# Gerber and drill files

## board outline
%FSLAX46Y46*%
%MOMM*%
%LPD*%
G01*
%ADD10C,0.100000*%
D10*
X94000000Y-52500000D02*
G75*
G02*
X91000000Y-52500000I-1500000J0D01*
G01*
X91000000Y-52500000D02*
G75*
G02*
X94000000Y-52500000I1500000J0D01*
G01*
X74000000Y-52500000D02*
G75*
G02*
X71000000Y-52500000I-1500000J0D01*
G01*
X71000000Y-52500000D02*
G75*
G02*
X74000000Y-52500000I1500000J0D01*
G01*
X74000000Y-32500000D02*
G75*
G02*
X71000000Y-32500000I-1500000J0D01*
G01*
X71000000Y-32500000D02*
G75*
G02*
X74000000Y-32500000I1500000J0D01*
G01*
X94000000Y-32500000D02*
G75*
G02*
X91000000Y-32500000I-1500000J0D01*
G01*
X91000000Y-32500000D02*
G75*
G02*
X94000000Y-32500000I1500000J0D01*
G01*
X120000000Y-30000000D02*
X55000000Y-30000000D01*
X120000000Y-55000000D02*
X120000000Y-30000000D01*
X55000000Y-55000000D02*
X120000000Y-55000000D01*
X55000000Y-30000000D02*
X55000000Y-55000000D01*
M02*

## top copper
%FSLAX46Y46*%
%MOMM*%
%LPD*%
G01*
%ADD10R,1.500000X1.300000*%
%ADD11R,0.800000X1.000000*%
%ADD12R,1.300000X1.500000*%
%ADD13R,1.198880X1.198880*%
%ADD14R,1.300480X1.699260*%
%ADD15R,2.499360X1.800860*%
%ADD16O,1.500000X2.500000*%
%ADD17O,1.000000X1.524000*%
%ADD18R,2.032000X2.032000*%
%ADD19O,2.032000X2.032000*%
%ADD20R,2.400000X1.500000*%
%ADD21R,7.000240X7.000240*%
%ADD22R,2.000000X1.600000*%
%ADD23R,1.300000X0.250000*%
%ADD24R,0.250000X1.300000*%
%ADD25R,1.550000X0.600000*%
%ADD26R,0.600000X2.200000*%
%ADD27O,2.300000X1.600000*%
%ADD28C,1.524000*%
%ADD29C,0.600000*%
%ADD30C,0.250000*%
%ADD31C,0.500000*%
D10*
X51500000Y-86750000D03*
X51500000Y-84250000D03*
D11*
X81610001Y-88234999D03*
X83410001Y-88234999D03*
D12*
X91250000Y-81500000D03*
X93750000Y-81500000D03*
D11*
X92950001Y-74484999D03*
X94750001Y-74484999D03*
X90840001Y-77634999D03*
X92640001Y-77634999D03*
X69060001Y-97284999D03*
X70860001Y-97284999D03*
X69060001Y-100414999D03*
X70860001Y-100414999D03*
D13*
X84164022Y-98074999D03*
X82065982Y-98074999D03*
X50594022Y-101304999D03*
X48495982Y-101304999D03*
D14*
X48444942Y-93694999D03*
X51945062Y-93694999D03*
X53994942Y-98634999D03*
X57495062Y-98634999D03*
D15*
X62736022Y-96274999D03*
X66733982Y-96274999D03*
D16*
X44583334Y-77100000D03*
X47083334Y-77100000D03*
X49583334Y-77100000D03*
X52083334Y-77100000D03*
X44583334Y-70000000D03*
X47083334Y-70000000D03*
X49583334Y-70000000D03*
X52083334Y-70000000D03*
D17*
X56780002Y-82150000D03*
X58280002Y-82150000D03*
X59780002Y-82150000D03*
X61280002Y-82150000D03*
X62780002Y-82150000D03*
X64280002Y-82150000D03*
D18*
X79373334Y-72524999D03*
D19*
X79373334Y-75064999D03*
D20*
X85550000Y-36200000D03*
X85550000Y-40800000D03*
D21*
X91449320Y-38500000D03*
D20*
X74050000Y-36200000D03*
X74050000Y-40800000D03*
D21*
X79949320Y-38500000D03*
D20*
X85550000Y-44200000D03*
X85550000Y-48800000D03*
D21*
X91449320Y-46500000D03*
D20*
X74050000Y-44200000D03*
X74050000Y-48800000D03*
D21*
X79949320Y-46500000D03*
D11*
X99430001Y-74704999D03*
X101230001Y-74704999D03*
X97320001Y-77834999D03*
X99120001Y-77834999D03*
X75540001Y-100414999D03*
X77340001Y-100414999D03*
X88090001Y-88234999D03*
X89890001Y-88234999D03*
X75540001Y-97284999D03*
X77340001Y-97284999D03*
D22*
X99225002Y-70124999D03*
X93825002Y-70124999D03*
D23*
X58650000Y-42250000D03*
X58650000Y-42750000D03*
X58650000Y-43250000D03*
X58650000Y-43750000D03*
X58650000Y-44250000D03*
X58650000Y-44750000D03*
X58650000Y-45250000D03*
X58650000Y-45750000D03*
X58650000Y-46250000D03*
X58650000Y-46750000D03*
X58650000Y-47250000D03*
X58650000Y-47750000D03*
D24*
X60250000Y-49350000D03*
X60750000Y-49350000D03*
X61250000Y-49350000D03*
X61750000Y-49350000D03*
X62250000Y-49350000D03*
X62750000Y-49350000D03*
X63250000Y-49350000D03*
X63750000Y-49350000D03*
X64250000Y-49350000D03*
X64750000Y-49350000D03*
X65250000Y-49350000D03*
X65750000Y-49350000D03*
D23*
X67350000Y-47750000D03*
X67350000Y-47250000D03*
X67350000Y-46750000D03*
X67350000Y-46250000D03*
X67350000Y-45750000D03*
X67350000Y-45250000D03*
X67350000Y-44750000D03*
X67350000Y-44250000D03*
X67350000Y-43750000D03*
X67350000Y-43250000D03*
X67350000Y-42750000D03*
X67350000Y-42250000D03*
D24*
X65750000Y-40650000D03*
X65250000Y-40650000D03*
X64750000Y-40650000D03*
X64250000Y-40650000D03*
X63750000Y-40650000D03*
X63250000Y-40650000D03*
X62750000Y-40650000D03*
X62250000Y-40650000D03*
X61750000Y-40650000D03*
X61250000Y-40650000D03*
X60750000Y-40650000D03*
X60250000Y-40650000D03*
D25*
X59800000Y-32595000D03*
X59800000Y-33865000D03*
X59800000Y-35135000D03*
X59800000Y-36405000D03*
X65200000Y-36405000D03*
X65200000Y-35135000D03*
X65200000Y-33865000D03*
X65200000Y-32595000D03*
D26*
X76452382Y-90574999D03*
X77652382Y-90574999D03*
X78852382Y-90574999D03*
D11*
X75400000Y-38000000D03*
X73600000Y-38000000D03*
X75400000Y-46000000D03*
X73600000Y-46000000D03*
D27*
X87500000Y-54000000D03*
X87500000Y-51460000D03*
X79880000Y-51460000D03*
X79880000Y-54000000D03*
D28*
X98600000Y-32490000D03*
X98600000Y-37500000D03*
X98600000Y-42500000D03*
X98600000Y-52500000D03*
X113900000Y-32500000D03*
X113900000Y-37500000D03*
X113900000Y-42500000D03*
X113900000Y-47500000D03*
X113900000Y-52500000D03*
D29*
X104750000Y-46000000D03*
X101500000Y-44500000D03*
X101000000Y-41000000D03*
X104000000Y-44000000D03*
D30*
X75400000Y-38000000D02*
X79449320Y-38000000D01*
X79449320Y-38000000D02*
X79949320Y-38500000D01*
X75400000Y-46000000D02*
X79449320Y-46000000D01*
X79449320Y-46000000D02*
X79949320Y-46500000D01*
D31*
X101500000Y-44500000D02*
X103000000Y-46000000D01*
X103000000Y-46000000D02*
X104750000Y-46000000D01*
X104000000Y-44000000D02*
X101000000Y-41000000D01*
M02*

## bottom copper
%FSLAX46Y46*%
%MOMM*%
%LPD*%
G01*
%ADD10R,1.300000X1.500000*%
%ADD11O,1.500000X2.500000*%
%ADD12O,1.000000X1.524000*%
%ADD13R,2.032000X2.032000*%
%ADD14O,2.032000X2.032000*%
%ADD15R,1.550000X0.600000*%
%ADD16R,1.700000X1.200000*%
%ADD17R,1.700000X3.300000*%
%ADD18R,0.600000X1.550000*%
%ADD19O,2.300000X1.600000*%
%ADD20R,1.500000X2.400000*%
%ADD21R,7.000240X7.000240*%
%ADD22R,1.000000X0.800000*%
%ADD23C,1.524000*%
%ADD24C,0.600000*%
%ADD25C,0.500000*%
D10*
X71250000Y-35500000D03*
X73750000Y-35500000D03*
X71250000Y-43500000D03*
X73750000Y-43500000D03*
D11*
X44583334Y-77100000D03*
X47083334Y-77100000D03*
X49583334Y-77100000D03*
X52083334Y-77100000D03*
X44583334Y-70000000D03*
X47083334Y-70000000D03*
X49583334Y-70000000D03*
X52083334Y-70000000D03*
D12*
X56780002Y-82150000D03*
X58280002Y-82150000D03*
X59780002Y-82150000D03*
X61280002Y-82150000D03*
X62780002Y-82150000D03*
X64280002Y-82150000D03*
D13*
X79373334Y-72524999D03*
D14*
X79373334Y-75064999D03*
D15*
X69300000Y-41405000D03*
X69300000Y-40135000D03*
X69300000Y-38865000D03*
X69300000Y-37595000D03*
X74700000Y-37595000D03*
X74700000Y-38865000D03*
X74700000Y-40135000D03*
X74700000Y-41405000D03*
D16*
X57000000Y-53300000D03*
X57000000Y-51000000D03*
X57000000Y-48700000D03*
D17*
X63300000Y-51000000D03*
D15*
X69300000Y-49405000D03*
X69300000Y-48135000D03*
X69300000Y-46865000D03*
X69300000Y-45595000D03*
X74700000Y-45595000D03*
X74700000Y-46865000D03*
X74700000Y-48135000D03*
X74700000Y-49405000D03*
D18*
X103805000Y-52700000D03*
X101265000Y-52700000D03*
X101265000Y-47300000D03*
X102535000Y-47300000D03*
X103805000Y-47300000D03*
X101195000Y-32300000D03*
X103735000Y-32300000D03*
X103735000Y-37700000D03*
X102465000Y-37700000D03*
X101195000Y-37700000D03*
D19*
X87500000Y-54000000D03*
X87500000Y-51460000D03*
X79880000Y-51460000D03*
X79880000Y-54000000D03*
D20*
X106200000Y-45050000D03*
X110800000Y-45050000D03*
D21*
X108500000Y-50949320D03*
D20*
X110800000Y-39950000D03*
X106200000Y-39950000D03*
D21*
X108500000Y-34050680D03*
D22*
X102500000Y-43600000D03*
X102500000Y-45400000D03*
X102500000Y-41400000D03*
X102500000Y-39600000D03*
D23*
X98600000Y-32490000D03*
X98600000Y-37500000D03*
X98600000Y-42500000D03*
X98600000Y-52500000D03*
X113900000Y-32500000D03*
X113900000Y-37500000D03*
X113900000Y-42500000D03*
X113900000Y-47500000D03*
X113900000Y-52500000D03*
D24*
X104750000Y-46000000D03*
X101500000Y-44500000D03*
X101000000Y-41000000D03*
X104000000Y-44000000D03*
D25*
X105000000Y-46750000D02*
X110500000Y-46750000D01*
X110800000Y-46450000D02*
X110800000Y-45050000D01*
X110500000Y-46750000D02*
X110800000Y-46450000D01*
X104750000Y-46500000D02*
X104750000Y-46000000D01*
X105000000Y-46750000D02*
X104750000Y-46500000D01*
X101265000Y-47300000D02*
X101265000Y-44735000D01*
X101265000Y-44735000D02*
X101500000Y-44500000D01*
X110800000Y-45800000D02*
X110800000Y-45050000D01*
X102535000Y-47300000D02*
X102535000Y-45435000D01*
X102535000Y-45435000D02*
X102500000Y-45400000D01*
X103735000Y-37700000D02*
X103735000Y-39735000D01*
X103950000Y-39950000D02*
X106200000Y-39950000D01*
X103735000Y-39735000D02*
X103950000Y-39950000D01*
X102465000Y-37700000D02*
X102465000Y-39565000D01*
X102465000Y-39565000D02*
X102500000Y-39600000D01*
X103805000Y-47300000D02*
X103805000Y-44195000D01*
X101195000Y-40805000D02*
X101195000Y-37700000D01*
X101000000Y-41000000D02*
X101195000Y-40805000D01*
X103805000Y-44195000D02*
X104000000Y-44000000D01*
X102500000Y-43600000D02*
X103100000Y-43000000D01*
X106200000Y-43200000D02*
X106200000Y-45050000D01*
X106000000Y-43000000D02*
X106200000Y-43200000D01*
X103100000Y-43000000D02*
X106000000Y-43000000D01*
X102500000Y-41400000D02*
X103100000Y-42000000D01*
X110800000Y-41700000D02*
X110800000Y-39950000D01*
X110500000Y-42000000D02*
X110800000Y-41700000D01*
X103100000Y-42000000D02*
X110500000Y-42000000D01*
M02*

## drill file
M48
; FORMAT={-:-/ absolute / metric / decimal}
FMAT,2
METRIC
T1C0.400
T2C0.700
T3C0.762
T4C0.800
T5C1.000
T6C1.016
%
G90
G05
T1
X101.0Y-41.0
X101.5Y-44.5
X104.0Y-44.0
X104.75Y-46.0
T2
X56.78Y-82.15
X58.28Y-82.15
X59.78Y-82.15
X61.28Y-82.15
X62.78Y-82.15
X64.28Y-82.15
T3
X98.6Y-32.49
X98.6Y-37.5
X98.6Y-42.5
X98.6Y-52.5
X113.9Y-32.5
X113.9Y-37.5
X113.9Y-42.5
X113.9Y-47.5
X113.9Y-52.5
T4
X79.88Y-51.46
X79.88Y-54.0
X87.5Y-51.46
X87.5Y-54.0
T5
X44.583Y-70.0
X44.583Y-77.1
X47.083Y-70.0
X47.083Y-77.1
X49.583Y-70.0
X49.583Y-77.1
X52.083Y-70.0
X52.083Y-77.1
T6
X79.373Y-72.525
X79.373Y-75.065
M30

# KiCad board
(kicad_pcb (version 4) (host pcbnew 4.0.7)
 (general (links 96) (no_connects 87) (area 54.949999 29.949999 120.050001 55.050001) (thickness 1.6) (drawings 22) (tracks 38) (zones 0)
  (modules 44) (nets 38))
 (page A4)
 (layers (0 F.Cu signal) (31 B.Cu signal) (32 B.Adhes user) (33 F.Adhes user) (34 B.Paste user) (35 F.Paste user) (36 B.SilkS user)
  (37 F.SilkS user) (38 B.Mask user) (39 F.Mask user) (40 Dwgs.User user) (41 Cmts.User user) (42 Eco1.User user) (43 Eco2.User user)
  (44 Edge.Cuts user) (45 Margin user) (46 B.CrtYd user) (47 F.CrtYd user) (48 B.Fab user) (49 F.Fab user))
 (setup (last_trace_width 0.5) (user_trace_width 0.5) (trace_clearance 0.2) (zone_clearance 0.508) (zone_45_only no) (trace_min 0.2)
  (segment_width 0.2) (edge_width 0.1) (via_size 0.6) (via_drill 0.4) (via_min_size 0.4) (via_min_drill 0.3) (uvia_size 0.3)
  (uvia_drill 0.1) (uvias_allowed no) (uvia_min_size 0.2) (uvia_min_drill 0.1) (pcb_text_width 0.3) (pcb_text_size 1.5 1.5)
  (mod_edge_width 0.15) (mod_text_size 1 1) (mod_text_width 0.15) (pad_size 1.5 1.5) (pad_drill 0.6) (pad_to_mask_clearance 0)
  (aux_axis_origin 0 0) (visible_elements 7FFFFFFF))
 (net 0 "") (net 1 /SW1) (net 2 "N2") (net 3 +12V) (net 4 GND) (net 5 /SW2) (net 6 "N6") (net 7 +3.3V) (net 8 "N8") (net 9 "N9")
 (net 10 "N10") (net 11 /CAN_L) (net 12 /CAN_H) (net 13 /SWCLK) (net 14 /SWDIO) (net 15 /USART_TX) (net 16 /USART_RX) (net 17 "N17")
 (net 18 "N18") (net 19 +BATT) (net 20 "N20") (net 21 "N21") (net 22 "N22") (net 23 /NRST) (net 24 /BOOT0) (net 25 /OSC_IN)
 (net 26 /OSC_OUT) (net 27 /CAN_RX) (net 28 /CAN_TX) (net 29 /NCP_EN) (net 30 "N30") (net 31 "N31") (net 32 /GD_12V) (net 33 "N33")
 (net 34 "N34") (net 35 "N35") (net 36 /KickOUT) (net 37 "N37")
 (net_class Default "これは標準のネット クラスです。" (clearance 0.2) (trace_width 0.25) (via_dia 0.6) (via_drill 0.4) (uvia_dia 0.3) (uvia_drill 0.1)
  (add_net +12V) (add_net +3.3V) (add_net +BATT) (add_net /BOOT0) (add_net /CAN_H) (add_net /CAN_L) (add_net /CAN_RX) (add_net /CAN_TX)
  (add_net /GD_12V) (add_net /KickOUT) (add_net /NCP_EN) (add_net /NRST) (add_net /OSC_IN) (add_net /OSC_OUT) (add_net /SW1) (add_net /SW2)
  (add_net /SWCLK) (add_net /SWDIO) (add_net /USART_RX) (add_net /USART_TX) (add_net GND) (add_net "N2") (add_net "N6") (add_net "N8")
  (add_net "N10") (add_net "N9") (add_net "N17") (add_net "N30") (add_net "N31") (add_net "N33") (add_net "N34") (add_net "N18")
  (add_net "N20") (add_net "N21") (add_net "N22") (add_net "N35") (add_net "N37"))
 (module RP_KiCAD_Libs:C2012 (layer B.Cu) (at 72.5 35.5)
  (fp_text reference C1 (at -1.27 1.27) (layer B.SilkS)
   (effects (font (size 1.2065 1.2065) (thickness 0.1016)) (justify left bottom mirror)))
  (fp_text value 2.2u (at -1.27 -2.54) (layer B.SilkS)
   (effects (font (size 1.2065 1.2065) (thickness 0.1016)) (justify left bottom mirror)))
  (pad 1 smd rect (at -1.25 0) (size 1.3 1.5) (layers B.Cu B.Paste B.Mask) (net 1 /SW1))
  (pad 2 smd rect (at 1.25 0) (size 1.3 1.5) (layers B.Cu B.Paste B.Mask) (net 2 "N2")))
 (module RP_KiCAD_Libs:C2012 (layer F.Cu) (at 51.5 85.5 90)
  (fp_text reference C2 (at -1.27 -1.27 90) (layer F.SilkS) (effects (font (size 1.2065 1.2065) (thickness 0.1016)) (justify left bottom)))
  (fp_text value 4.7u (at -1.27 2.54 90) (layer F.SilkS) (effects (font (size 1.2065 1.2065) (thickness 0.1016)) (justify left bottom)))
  (pad 1 smd rect (at -1.25 0 90) (size 1.3 1.5) (layers F.Cu F.Paste F.Mask) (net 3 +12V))
  (pad 2 smd rect (at 1.25 0 90) (size 1.3 1.5) (layers F.Cu F.Paste F.Mask) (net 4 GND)))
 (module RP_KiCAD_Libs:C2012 (layer B.Cu) (at 72.5 43.5)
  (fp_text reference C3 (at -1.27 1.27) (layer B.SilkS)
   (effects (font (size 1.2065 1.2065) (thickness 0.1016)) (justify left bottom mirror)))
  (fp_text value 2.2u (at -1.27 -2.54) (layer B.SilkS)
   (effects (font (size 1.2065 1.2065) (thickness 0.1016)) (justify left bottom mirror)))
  (pad 1 smd rect (at -1.25 0) (size 1.3 1.5) (layers B.Cu B.Paste B.Mask) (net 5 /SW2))
  (pad 2 smd rect (at 1.25 0) (size 1.3 1.5) (layers B.Cu B.Paste B.Mask) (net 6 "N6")))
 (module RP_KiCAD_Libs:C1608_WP (layer F.Cu) (at 82.510001 88.234999)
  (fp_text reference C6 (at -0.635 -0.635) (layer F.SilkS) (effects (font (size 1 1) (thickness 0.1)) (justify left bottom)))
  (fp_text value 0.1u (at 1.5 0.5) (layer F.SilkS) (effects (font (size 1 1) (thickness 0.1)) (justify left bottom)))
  (pad 1 smd rect (at -0.9 0) (size 0.8 1) (layers F.Cu F.Paste F.Mask) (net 4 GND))
  (pad 2 smd rect (at 0.9 0) (size 0.8 1) (layers F.Cu F.Paste F.Mask) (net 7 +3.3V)))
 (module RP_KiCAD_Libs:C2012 (layer F.Cu) (at 92.5 81.5)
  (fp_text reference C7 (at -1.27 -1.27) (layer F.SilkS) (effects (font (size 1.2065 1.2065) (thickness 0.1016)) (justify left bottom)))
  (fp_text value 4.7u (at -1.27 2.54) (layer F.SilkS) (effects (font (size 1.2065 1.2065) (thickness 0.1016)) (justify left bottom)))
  (pad 1 smd rect (at -1.25 0) (size 1.3 1.5) (layers F.Cu F.Paste F.Mask) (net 7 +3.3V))
  (pad 2 smd rect (at 1.25 0) (size 1.3 1.5) (layers F.Cu F.Paste F.Mask) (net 4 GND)))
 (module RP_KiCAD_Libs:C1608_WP (layer F.Cu) (at 93.850001 74.484999)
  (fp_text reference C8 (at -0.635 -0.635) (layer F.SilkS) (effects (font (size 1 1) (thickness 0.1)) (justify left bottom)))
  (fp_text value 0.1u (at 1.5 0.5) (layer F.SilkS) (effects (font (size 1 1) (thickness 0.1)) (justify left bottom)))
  (pad 1 smd rect (at -0.9 0) (size 0.8 1) (layers F.Cu F.Paste F.Mask) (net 4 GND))
  (pad 2 smd rect (at 0.9 0) (size 0.8 1) (layers F.Cu F.Paste F.Mask) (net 7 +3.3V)))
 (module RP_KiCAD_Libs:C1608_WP (layer F.Cu) (at 91.740001 77.634999)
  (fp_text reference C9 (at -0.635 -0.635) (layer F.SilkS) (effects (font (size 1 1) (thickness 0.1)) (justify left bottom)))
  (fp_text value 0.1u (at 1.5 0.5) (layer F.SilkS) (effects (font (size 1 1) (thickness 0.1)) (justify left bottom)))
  (pad 1 smd rect (at -0.9 0) (size 0.8 1) (layers F.Cu F.Paste F.Mask) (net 4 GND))
  (pad 2 smd rect (at 0.9 0) (size 0.8 1) (layers F.Cu F.Paste F.Mask) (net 7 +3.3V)))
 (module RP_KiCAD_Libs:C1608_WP (layer F.Cu) (at 69.960001 97.284999)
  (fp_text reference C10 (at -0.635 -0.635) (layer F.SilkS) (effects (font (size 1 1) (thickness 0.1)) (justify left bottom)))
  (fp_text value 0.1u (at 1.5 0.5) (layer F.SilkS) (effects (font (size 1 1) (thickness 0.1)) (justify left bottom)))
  (pad 1 smd rect (at -0.9 0) (size 0.8 1) (layers F.Cu F.Paste F.Mask) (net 4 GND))
  (pad 2 smd rect (at 0.9 0) (size 0.8 1) (layers F.Cu F.Paste F.Mask) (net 7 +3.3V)))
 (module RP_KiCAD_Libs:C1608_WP (layer F.Cu) (at 69.960001 100.414999)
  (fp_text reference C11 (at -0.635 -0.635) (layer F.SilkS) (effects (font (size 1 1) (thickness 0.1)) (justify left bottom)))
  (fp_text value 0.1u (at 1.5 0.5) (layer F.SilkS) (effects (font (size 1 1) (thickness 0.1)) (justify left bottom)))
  (pad 1 smd rect (at -0.9 0) (size 0.8 1) (layers F.Cu F.Paste F.Mask) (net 4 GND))
  (pad 2 smd rect (at 0.9 0) (size 0.8 1) (layers F.Cu F.Paste F.Mask) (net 7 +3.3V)))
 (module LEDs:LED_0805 (layer F.Cu) (at 83.115002 98.074999)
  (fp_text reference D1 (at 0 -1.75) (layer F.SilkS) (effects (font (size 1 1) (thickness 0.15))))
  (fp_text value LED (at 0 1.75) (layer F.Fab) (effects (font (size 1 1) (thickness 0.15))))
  (pad 1 smd rect (at 1.04902 0 180) (size 1.19888 1.19888) (layers F.Cu F.Paste F.Mask) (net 7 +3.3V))
  (pad 2 smd rect (at -1.04902 0 180) (size 1.19888 1.19888) (layers F.Cu F.Paste F.Mask) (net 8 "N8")))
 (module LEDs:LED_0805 (layer F.Cu) (at 49.545002 101.304999)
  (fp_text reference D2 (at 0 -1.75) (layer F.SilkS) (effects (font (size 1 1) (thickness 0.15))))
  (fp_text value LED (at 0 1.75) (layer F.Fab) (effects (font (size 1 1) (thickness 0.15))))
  (pad 1 smd rect (at 1.04902 0 180) (size 1.19888 1.19888) (layers F.Cu F.Paste F.Mask))
  (pad 2 smd rect (at -1.04902 0 180) (size 1.19888 1.19888) (layers F.Cu F.Paste F.Mask) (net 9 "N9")))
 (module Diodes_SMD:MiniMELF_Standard (layer F.Cu) (at 50.195002 93.694999)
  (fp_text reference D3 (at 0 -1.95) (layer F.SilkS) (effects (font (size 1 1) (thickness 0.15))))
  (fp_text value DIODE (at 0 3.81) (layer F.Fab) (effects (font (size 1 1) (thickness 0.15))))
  (pad 1 smd rect (at -1.75006 0) (size 1.30048 1.69926) (layers F.Cu F.Paste F.Mask) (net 2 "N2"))
  (pad 2 smd rect (at 1.75006 0) (size 1.30048 1.69926) (layers F.Cu F.Paste F.Mask) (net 3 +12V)))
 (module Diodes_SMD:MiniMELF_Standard (layer F.Cu) (at 55.745002 98.634999)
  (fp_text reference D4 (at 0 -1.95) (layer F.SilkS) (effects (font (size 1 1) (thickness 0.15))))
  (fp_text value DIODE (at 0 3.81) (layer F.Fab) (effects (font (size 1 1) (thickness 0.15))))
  (pad 1 smd rect (at -1.75006 0) (size 1.30048 1.69926) (layers F.Cu F.Paste F.Mask) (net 6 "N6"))
  (pad 2 smd rect (at 1.75006 0) (size 1.30048 1.69926) (layers F.Cu F.Paste F.Mask) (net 3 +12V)))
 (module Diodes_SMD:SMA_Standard (layer F.Cu) (at 64.735002 96.274999)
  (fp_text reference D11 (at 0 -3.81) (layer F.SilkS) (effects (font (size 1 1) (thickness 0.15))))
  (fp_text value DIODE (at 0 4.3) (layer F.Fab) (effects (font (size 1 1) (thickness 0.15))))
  (pad 1 smd rect (at -1.99898 0) (size 2.49936 1.80086) (layers F.Cu F.Paste F.Mask) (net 3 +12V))
  (pad 2 smd rect (at 1.99898 0) (size 2.49936 1.80086) (layers F.Cu F.Paste F.Mask) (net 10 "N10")))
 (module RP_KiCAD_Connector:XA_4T (layer F.Cu) (at 44.583334 77.1)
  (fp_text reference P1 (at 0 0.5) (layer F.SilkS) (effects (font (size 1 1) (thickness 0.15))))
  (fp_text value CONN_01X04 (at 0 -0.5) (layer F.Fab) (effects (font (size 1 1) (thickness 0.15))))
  (pad 4 thru_hole oval (at 0 0) (size 1.5 2.5) (drill 1) (layers *.Cu *.Mask F.SilkS) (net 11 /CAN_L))
  (pad 3 thru_hole oval (at 2.5 0) (size 1.5 2.5) (drill 1) (layers *.Cu *.Mask F.SilkS) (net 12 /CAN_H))
  (pad 2 thru_hole oval (at 5 0) (size 1.5 2.5) (drill 1) (layers *.Cu *.Mask F.SilkS) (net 10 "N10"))
  (pad 1 thru_hole oval (at 7.5 0) (size 1.5 2.5) (drill 1) (layers *.Cu *.Mask F.SilkS) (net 4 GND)))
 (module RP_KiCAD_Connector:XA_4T (layer F.Cu) (at 44.583334 70)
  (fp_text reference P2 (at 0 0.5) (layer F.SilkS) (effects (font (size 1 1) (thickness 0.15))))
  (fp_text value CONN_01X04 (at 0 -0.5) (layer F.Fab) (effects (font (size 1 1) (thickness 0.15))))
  (pad 4 thru_hole oval (at 0 0) (size 1.5 2.5) (drill 1) (layers *.Cu *.Mask F.SilkS) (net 11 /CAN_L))
  (pad 3 thru_hole oval (at 2.5 0) (size 1.5 2.5) (drill 1) (layers *.Cu *.Mask F.SilkS) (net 12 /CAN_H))
  (pad 2 thru_hole oval (at 5 0) (size 1.5 2.5) (drill 1) (layers *.Cu *.Mask F.SilkS) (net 10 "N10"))
  (pad 1 thru_hole oval (at 7.5 0) (size 1.5 2.5) (drill 1) (layers *.Cu *.Mask F.SilkS) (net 4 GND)))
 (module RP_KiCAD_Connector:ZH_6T (layer F.Cu) (at 56.780002 82.15)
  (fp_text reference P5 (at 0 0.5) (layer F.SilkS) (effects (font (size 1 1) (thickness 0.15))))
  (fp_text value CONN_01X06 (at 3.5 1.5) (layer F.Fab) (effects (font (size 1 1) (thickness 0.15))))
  (pad 1 thru_hole oval (at 0 0) (size 1 1.524) (drill 0.7) (layers *.Cu *.Mask) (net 4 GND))
  (pad 2 thru_hole oval (at 1.5 0) (size 1 1.524) (drill 0.7) (layers *.Cu *.Mask))
  (pad 3 thru_hole oval (at 3 0) (size 1 1.524) (drill 0.7) (layers *.Cu *.Mask) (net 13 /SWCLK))
  (pad 4 thru_hole oval (at 4.5 0) (size 1 1.524) (drill 0.7) (layers *.Cu *.Mask) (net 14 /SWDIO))
  (pad 5 thru_hole oval (at 6 0) (size 1 1.524) (drill 0.7) (layers *.Cu *.Mask) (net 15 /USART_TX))
  (pad 6 thru_hole oval (at 7.5 0) (size 1 1.524) (drill 0.7) (layers *.Cu *.Mask) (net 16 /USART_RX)))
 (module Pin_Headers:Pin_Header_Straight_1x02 (layer F.Cu) (at 79.373334 72.524999)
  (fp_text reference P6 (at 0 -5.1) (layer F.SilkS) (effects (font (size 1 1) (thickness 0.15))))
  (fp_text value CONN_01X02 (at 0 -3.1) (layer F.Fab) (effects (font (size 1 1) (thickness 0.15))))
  (pad 1 thru_hole rect (at 0 0) (size 2.032 2.032) (drill 1.016) (layers *.Cu *.Mask F.SilkS) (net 12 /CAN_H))
  (pad 2 thru_hole oval (at 0 2.54) (size 2.032 2.032) (drill 1.016) (layers *.Cu *.Mask F.SilkS) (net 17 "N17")))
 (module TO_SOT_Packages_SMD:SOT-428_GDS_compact (layer F.Cu) (at 89 38.5 270)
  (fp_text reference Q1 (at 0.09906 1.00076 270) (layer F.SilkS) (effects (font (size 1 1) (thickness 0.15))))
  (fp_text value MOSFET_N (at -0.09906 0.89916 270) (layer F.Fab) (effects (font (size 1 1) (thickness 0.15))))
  (pad G smd rect (at -2.3 3.45 270) (size 1.5 2.4) (layers F.Cu F.Paste F.Mask) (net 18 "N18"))
  (pad S smd rect (at 2.3 3.45 270) (size 1.5 2.4) (layers F.Cu F.Paste F.Mask) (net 1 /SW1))
  (pad D smd rect (at 0 -2.44932 270) (size 7.00024 7.00024) (layers F.Cu F.Paste F.Mask) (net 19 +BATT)))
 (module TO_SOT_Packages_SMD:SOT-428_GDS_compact (layer F.Cu) (at 77.5 38.5 270)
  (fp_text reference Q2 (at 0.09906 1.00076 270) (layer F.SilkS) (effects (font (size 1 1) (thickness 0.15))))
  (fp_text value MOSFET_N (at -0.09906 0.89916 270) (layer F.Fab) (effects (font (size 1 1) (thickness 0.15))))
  (pad G smd rect (at -2.3 3.45 270) (size 1.5 2.4) (layers F.Cu F.Paste F.Mask) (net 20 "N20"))
  (pad S smd rect (at 2.3 3.45 270) (size 1.5 2.4) (layers F.Cu F.Paste F.Mask) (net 4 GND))
  (pad D smd rect (at 0 -2.44932 270) (size 7.00024 7.00024) (layers F.Cu F.Paste F.Mask) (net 1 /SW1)))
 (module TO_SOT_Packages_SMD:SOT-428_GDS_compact (layer F.Cu) (at 89 46.5 270)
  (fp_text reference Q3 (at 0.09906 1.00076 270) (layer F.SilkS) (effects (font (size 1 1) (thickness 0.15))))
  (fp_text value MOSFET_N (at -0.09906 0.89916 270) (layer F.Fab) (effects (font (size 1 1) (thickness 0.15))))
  (pad G smd rect (at -2.3 3.45 270) (size 1.5 2.4) (layers F.Cu F.Paste F.Mask) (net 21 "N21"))
  (pad S smd rect (at 2.3 3.45 270) (size 1.5 2.4) (layers F.Cu F.Paste F.Mask) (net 5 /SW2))
  (pad D smd rect (at 0 -2.44932 270) (size 7.00024 7.00024) (layers F.Cu F.Paste F.Mask) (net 19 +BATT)))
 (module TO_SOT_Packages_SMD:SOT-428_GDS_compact (layer F.Cu) (at 77.5 46.5 270)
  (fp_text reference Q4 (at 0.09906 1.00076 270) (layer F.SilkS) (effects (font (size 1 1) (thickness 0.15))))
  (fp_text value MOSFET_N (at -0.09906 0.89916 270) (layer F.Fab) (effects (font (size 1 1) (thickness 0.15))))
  (pad G smd rect (at -2.3 3.45 270) (size 1.5 2.4) (layers F.Cu F.Paste F.Mask) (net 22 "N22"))
  (pad S smd rect (at 2.3 3.45 270) (size 1.5 2.4) (layers F.Cu F.Paste F.Mask) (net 4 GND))
  (pad D smd rect (at 0 -2.44932 270) (size 7.00024 7.00024) (layers F.Cu F.Paste F.Mask) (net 5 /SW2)))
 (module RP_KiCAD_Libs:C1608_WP (layer F.Cu) (at 100.330001 74.704999)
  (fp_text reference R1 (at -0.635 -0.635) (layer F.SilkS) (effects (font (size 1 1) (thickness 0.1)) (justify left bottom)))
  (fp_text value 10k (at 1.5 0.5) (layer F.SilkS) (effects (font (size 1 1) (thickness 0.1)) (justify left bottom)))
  (pad 1 smd rect (at -0.9 0) (size 0.8 1) (layers F.Cu F.Paste F.Mask) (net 7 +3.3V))
  (pad 2 smd rect (at 0.9 0) (size 0.8 1) (layers F.Cu F.Paste F.Mask) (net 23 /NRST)))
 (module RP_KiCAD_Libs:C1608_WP (layer F.Cu) (at 98.220001 77.834999)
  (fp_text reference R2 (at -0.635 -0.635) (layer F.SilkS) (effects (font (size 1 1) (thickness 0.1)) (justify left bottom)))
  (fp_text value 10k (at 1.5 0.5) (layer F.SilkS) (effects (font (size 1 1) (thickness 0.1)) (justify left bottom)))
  (pad 1 smd rect (at -0.9 0) (size 0.8 1) (layers F.Cu F.Paste F.Mask) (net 4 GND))
  (pad 2 smd rect (at 0.9 0) (size 0.8 1) (layers F.Cu F.Paste F.Mask) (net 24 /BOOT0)))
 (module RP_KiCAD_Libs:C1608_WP (layer F.Cu) (at 76.440001 100.414999)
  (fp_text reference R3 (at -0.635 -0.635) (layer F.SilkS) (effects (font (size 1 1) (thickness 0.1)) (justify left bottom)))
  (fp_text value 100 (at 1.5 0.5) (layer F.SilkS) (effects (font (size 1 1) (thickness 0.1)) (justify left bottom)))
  (pad 1 smd rect (at -0.9 0) (size 0.8 1) (layers F.Cu F.Paste F.Mask) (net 8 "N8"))
  (pad 2 smd rect (at 0.9 0) (size 0.8 1) (layers F.Cu F.Paste F.Mask) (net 4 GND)))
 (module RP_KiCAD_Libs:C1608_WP (layer F.Cu) (at 88.990001 88.234999)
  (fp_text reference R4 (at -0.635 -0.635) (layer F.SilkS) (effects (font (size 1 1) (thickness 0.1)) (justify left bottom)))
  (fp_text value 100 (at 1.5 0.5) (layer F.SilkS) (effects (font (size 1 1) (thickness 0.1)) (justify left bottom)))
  (pad 1 smd rect (at -0.9 0) (size 0.8 1) (layers F.Cu F.Paste F.Mask) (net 9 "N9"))
  (pad 2 smd rect (at 0.9 0) (size 0.8 1) (layers F.Cu F.Paste F.Mask) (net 4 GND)))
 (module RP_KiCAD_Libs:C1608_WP (layer F.Cu) (at 76.440001 97.284999)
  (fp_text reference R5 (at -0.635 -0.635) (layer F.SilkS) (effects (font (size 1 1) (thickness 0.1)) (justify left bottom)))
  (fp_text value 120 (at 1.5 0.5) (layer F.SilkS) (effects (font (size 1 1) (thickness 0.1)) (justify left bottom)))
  (pad 1 smd rect (at -0.9 0) (size 0.8 1) (layers F.Cu F.Paste F.Mask) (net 11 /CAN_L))
  (pad 2 smd rect (at 0.9 0) (size 0.8 1) (layers F.Cu F.Paste F.Mask) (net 17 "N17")))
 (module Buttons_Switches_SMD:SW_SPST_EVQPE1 (layer F.Cu) (at 96.525002 70.124999)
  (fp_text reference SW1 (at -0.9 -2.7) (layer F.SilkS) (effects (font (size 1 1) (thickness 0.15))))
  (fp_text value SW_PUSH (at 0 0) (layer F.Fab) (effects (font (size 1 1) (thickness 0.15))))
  (pad 2 smd rect (at 2.7 0) (size 2 1.6) (layers F.Cu F.Paste F.Mask) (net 23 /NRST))
  (pad 1 smd rect (at -2.7 0) (size 2 1.6) (layers F.Cu F.Paste F.Mask) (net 4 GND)))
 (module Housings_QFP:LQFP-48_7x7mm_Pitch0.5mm (layer F.Cu) (at 63 45)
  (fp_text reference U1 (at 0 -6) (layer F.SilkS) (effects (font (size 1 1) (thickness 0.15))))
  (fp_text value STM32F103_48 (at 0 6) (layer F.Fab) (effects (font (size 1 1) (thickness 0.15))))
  (pad 1 smd rect (at -4.35 -2.75) (size 1.3 0.25) (layers F.Cu F.Paste F.Mask))
  (pad 2 smd rect (at -4.35 -2.25) (size 1.3 0.25) (layers F.Cu F.Paste F.Mask))
  (pad 3 smd rect (at -4.35 -1.75) (size 1.3 0.25) (layers F.Cu F.Paste F.Mask))
  (pad 4 smd rect (at -4.35 -1.25) (size 1.3 0.25) (layers F.Cu F.Paste F.Mask))
  (pad 5 smd rect (at -4.35 -0.75) (size 1.3 0.25) (layers F.Cu F.Paste F.Mask) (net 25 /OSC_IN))
  (pad 6 smd rect (at -4.35 -0.25) (size 1.3 0.25) (layers F.Cu F.Paste F.Mask) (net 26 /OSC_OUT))
  (pad 7 smd rect (at -4.35 0.25) (size 1.3 0.25) (layers F.Cu F.Paste F.Mask) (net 23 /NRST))
  (pad 8 smd rect (at -4.35 0.75) (size 1.3 0.25) (layers F.Cu F.Paste F.Mask) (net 4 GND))
  (pad 9 smd rect (at -4.35 1.25) (size 1.3 0.25) (layers F.Cu F.Paste F.Mask) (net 7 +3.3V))
  (pad 10 smd rect (at -4.35 1.75) (size 1.3 0.25) (layers F.Cu F.Paste F.Mask))
  (pad 11 smd rect (at -4.35 2.25) (size 1.3 0.25) (layers F.Cu F.Paste F.Mask))
  (pad 12 smd rect (at -4.35 2.75) (size 1.3 0.25) (layers F.Cu F.Paste F.Mask))
  (pad 13 smd rect (at -2.75 4.35 90) (size 1.3 0.25) (layers F.Cu F.Paste F.Mask))
  (pad 14 smd rect (at -2.25 4.35 90) (size 1.3 0.25) (layers F.Cu F.Paste F.Mask))
  (pad 15 smd rect (at -1.75 4.35 90) (size 1.3 0.25) (layers F.Cu F.Paste F.Mask))
  (pad 16 smd rect (at -1.25 4.35 90) (size 1.3 0.25) (layers F.Cu F.Paste F.Mask))
  (pad 17 smd rect (at -0.75 4.35 90) (size 1.3 0.25) (layers F.Cu F.Paste F.Mask))
  (pad 18 smd rect (at -0.25 4.35 90) (size 1.3 0.25) (layers F.Cu F.Paste F.Mask))
  (pad 19 smd rect (at 0.25 4.35 90) (size 1.3 0.25) (layers F.Cu F.Paste F.Mask))
  (pad 20 smd rect (at 0.75 4.35 90) (size 1.3 0.25) (layers F.Cu F.Paste F.Mask))
  (pad 21 smd rect (at 1.25 4.35 90) (size 1.3 0.25) (layers F.Cu F.Paste F.Mask))
  (pad 22 smd rect (at 1.75 4.35 90) (size 1.3 0.25) (layers F.Cu F.Paste F.Mask))
  (pad 23 smd rect (at 2.25 4.35 90) (size 1.3 0.25) (layers F.Cu F.Paste F.Mask) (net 4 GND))
  (pad 24 smd rect (at 2.75 4.35 90) (size 1.3 0.25) (layers F.Cu F.Paste F.Mask) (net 7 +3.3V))
  (pad 25 smd rect (at 4.35 2.75) (size 1.3 0.25) (layers F.Cu F.Paste F.Mask))
  (pad 26 smd rect (at 4.35 2.25) (size 1.3 0.25) (layers F.Cu F.Paste F.Mask))
  (pad 27 smd rect (at 4.35 1.75) (size 1.3 0.25) (layers F.Cu F.Paste F.Mask))
  (pad 28 smd rect (at 4.35 1.25) (size 1.3 0.25) (layers F.Cu F.Paste F.Mask))
  (pad 29 smd rect (at 4.35 0.75) (size 1.3 0.25) (layers F.Cu F.Paste F.Mask))
  (pad 30 smd rect (at 4.35 0.25) (size 1.3 0.25) (layers F.Cu F.Paste F.Mask) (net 15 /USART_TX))
  (pad 31 smd rect (at 4.35 -0.25) (size 1.3 0.25) (layers F.Cu F.Paste F.Mask) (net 16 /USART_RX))
  (pad 32 smd rect (at 4.35 -0.75) (size 1.3 0.25) (layers F.Cu F.Paste F.Mask) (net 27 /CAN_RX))
  (pad 33 smd rect (at 4.35 -1.25) (size 1.3 0.25) (layers F.Cu F.Paste F.Mask) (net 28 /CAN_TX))
  (pad 34 smd rect (at 4.35 -1.75) (size 1.3 0.25) (layers F.Cu F.Paste F.Mask) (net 14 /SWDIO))
  (pad 35 smd rect (at 4.35 -2.25) (size 1.3 0.25) (layers F.Cu F.Paste F.Mask) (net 4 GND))
  (pad 36 smd rect (at 4.35 -2.75) (size 1.3 0.25) (layers F.Cu F.Paste F.Mask) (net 7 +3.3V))
  (pad 37 smd rect (at 2.75 -4.35 90) (size 1.3 0.25) (layers F.Cu F.Paste F.Mask) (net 13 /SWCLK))
  (pad 38 smd rect (at 2.25 -4.35 90) (size 1.3 0.25) (layers F.Cu F.Paste F.Mask))
  (pad 39 smd rect (at 1.75 -4.35 90) (size 1.3 0.25) (layers F.Cu F.Paste F.Mask))
  (pad 40 smd rect (at 1.25 -4.35 90) (size 1.3 0.25) (layers F.Cu F.Paste F.Mask))
  (pad 41 smd rect (at 0.75 -4.35 90) (size 1.3 0.25) (layers F.Cu F.Paste F.Mask))
  (pad 42 smd rect (at 0.25 -4.35 90) (size 1.3 0.25) (layers F.Cu F.Paste F.Mask))
  (pad 43 smd rect (at -0.25 -4.35 90) (size 1.3 0.25) (layers F.Cu F.Paste F.Mask))
  (pad 44 smd rect (at -0.75 -4.35 90) (size 1.3 0.25) (layers F.Cu F.Paste F.Mask) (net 24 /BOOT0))
  (pad 45 smd rect (at -1.25 -4.35 90) (size 1.3 0.25) (layers F.Cu F.Paste F.Mask))
  (pad 46 smd rect (at -1.75 -4.35 90) (size 1.3 0.25) (layers F.Cu F.Paste F.Mask))
  (pad 47 smd rect (at -2.25 -4.35 90) (size 1.3 0.25) (layers F.Cu F.Paste F.Mask) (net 4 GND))
  (pad 48 smd rect (at -2.75 -4.35 90) (size 1.3 0.25) (layers F.Cu F.Paste F.Mask) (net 7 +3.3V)))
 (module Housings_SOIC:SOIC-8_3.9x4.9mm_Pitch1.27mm (layer B.Cu) (at 72 39.5)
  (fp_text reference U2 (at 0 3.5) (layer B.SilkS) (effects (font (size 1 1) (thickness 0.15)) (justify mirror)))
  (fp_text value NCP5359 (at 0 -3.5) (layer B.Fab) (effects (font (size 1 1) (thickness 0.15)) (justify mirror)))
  (pad 1 smd rect (at -2.7 1.905) (size 1.55 0.6) (layers B.Cu B.Paste B.Mask) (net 3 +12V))
  (pad 2 smd rect (at -2.7 0.635) (size 1.55 0.6) (layers B.Cu B.Paste B.Mask))
  (pad 3 smd rect (at -2.7 -0.635) (size 1.55 0.6) (layers B.Cu B.Paste B.Mask) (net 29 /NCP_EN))
  (pad 4 smd rect (at -2.7 -1.905) (size 1.55 0.6) (layers B.Cu B.Paste B.Mask) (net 3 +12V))
  (pad 5 smd rect (at 2.7 -1.905) (size 1.55 0.6) (layers B.Cu B.Paste B.Mask) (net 20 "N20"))
  (pad 6 smd rect (at 2.7 -0.635) (size 1.55 0.6) (layers B.Cu B.Paste B.Mask) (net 4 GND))
  (pad 7 smd rect (at 2.7 0.635) (size 1.55 0.6) (layers B.Cu B.Paste B.Mask) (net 1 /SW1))
  (pad 8 smd rect (at 2.7 1.905) (size 1.55 0.6) (layers B.Cu B.Paste B.Mask) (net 18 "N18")))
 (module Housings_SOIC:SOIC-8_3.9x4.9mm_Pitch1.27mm (layer F.Cu) (at 62.5 34.5)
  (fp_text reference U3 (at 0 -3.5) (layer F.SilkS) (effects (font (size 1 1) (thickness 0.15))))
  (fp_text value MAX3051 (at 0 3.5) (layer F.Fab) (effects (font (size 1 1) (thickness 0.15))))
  (pad 1 smd rect (at -2.7 -1.905) (size 1.55 0.6) (layers F.Cu F.Paste F.Mask) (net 28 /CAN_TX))
  (pad 2 smd rect (at -2.7 -0.635) (size 1.55 0.6) (layers F.Cu F.Paste F.Mask) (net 4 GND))
  (pad 3 smd rect (at -2.7 0.635) (size 1.55 0.6) (layers F.Cu F.Paste F.Mask) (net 7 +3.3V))
  (pad 4 smd rect (at -2.7 1.905) (size 1.55 0.6) (layers F.Cu F.Paste F.Mask) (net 27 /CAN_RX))
  (pad 5 smd rect (at 2.7 1.905) (size 1.55 0.6) (layers F.Cu F.Paste F.Mask) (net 4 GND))
  (pad 6 smd rect (at 2.7 0.635) (size 1.55 0.6) (layers F.Cu F.Paste F.Mask) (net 11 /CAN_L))
  (pad 7 smd rect (at 2.7 -0.635) (size 1.55 0.6) (layers F.Cu F.Paste F.Mask) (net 12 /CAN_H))
  (pad 8 smd rect (at 2.7 -1.905) (size 1.55 0.6) (layers F.Cu F.Paste F.Mask) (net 4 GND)))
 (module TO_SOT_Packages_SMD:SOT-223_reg (layer B.Cu) (at 57 51 90)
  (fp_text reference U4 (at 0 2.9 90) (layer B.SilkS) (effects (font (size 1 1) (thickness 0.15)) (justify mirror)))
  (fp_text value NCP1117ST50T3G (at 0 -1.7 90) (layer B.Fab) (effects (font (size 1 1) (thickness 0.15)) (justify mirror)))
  (pad 1 smd rect (at -2.3 0 90) (size 1.2 1.7) (layers B.Cu B.Paste B.Mask) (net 4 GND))
  (pad 2 smd rect (at 0 0 90) (size 1.2 1.7) (layers B.Cu B.Paste B.Mask) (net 7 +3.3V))
  (pad 3 smd rect (at 2.3 0 90) (size 1.2 1.7) (layers B.Cu B.Paste B.Mask) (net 3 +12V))
  (pad 2 smd rect (at 0 6.3 90) (size 3.3 1.7) (layers B.Cu B.Paste B.Mask) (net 7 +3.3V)))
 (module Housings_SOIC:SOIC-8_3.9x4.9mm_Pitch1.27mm (layer B.Cu) (at 72 47.5)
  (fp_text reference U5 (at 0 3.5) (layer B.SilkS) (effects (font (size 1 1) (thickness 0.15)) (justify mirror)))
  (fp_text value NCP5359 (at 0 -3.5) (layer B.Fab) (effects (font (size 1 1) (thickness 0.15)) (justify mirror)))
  (pad 1 smd rect (at -2.7 1.905) (size 1.55 0.6) (layers B.Cu B.Paste B.Mask) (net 3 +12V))
  (pad 2 smd rect (at -2.7 0.635) (size 1.55 0.6) (layers B.Cu B.Paste B.Mask))
  (pad 3 smd rect (at -2.7 -0.635) (size 1.55 0.6) (layers B.Cu B.Paste B.Mask) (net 29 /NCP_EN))
  (pad 4 smd rect (at -2.7 -1.905) (size 1.55 0.6) (layers B.Cu B.Paste B.Mask) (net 3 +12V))
  (pad 5 smd rect (at 2.7 -1.905) (size 1.55 0.6) (layers B.Cu B.Paste B.Mask) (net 22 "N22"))
  (pad 6 smd rect (at 2.7 -0.635) (size 1.55 0.6) (layers B.Cu B.Paste B.Mask) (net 4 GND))
  (pad 7 smd rect (at 2.7 0.635) (size 1.55 0.6) (layers B.Cu B.Paste B.Mask) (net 5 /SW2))
  (pad 8 smd rect (at 2.7 1.905) (size 1.55 0.6) (layers B.Cu B.Paste B.Mask) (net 21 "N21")))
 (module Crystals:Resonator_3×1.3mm (layer F.Cu) (at 77.652382 90.574999)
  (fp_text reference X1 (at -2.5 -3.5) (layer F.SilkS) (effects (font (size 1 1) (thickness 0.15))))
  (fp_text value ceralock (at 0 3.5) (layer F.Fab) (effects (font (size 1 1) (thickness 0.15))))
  (pad 1 smd rect (at -1.2 0) (size 0.6 2.2) (layers F.Cu F.Paste F.Mask) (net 25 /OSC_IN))
  (pad 2 smd rect (at 0 0) (size 0.6 2.2) (layers F.Cu F.Paste F.Mask) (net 4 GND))
  (pad 3 smd rect (at 1.2 0) (size 0.6 2.2) (layers F.Cu F.Paste F.Mask) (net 26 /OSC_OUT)))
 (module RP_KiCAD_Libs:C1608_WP (layer F.Cu) (at 74.5 38 180)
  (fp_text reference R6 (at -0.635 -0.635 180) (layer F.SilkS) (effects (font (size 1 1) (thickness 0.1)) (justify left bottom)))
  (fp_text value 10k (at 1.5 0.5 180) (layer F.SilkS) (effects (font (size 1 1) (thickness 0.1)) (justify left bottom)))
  (pad 1 smd rect (at -0.9 0 180) (size 0.8 1) (layers F.Cu F.Paste F.Mask) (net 1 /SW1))
  (pad 2 smd rect (at 0.9 0 180) (size 0.8 1) (layers F.Cu F.Paste F.Mask) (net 4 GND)))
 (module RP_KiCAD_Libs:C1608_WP (layer F.Cu) (at 74.5 46 180)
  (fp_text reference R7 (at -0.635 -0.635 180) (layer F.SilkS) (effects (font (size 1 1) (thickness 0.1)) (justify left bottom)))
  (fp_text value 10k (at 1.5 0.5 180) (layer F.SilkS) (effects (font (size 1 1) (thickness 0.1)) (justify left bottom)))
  (pad 1 smd rect (at -0.9 0 180) (size 0.8 1) (layers F.Cu F.Paste F.Mask) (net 5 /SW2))
  (pad 2 smd rect (at 0.9 0 180) (size 0.8 1) (layers F.Cu F.Paste F.Mask) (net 4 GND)))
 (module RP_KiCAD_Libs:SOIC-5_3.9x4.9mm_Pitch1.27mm (layer B.Cu) (at 102.5 50 90)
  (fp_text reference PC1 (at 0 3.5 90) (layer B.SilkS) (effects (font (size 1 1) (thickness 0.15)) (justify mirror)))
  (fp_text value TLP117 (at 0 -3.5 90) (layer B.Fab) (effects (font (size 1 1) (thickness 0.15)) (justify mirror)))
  (pad 1 smd rect (at -2.7 1.305 90) (size 1.55 0.6) (layers B.Cu B.Paste B.Mask))
  (pad 3 smd rect (at -2.7 -1.235 90) (size 1.55 0.6) (layers B.Cu B.Paste B.Mask))
  (pad 4 smd rect (at 2.7 -1.235 90) (size 1.55 0.6) (layers B.Cu B.Paste B.Mask) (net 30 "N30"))
  (pad 5 smd rect (at 2.7 0.035 90) (size 1.55 0.6) (layers B.Cu B.Paste B.Mask) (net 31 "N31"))
  (pad 6 smd rect (at 2.7 1.305 90) (size 1.55 0.6) (layers B.Cu B.Paste B.Mask) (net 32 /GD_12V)))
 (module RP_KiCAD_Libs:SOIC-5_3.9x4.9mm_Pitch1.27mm (layer B.Cu) (at 102.5 35 270)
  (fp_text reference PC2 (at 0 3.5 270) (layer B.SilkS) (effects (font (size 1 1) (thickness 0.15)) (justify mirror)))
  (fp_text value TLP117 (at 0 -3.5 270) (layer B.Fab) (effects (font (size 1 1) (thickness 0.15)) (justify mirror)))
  (pad 1 smd rect (at -2.7 1.305 270) (size 1.55 0.6) (layers B.Cu B.Paste B.Mask))
  (pad 3 smd rect (at -2.7 -1.235 270) (size 1.55 0.6) (layers B.Cu B.Paste B.Mask))
  (pad 4 smd rect (at 2.7 -1.235 270) (size 1.55 0.6) (layers B.Cu B.Paste B.Mask) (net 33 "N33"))
  (pad 5 smd rect (at 2.7 0.035 270) (size 1.55 0.6) (layers B.Cu B.Paste B.Mask) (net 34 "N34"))
  (pad 6 smd rect (at 2.7 1.305 270) (size 1.55 0.6) (layers B.Cu B.Paste B.Mask) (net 32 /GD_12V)))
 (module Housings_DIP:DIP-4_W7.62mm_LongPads (layer F.Cu) (at 87.5 54 180)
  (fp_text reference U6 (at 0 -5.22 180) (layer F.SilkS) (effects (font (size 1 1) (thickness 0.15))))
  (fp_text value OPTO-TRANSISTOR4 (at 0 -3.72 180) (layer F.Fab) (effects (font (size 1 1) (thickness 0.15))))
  (pad 1 thru_hole oval (at 0 0 180) (size 2.3 1.6) (drill 0.8) (layers *.Cu *.Mask F.SilkS))
  (pad 2 thru_hole oval (at 0 2.54 180) (size 2.3 1.6) (drill 0.8) (layers *.Cu *.Mask F.SilkS))
  (pad 3 thru_hole oval (at 7.62 2.54 180) (size 2.3 1.6) (drill 0.8) (layers *.Cu *.Mask F.SilkS))
  (pad 4 thru_hole oval (at 7.62 0 180) (size 2.3 1.6) (drill 0.8) (layers *.Cu *.Mask F.SilkS)))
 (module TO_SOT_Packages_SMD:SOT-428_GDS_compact (layer B.Cu) (at 108.5 48.5)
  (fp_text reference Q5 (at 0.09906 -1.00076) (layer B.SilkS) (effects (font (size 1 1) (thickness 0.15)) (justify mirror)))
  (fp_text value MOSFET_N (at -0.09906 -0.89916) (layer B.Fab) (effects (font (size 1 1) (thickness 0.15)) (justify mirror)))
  (pad G smd rect (at -2.3 -3.45) (size 1.5 2.4) (layers B.Cu B.Paste B.Mask) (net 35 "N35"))
  (pad S smd rect (at 2.3 -3.45) (size 1.5 2.4) (layers B.Cu B.Paste B.Mask) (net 30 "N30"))
  (pad D smd rect (at 0 2.44932) (size 7.00024 7.00024) (layers B.Cu B.Paste B.Mask) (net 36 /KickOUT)))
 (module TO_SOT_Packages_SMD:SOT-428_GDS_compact (layer B.Cu) (at 108.5 36.5 180)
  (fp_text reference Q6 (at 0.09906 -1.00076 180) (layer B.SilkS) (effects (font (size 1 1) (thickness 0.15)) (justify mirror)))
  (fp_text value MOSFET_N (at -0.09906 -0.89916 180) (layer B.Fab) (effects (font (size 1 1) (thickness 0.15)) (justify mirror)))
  (pad G smd rect (at -2.3 -3.45 180) (size 1.5 2.4) (layers B.Cu B.Paste B.Mask) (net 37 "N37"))
  (pad S smd rect (at 2.3 -3.45 180) (size 1.5 2.4) (layers B.Cu B.Paste B.Mask) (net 33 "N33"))
  (pad D smd rect (at 0 2.44932 180) (size 7.00024 7.00024) (layers B.Cu B.Paste B.Mask) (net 36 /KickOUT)))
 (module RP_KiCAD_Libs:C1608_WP (layer B.Cu) (at 102.5 44.5 270)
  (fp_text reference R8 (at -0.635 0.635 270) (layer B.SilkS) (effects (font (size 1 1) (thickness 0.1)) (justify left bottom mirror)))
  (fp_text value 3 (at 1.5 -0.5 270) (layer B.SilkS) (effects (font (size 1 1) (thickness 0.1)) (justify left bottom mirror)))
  (pad 1 smd rect (at -0.9 0 270) (size 0.8 1) (layers B.Cu B.Paste B.Mask) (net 35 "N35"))
  (pad 2 smd rect (at 0.9 0 270) (size 0.8 1) (layers B.Cu B.Paste B.Mask) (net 31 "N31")))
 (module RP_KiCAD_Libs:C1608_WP (layer B.Cu) (at 102.5 40.5 90)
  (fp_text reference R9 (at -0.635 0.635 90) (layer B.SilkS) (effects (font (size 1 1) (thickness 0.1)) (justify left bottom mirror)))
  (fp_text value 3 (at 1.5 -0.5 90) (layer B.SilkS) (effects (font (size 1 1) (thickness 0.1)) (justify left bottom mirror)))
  (pad 1 smd rect (at -0.9 0 90) (size 0.8 1) (layers B.Cu B.Paste B.Mask) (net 37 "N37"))
  (pad 2 smd rect (at 0.9 0 90) (size 0.8 1) (layers B.Cu B.Paste B.Mask) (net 34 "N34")))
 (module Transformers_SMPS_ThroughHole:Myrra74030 (layer F.Cu) (at 95 29.25)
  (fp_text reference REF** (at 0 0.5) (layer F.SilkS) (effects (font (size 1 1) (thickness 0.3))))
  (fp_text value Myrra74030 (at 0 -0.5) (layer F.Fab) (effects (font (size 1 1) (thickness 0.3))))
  (pad 1 thru_hole circle (at 3.6 3.24) (size 1.524 1.524) (drill 0.762) (layers *.Cu *.Mask))
  (pad 2 thru_hole circle (at 3.6 8.25) (size 1.524 1.524) (drill 0.762) (layers *.Cu *.Mask))
  (pad 3 thru_hole circle (at 3.6 13.25) (size 1.524 1.524) (drill 0.762) (layers *.Cu *.Mask))
  (pad 5 thru_hole circle (at 3.6 23.25) (size 1.524 1.524) (drill 0.762) (layers *.Cu *.Mask))
  (pad 10 thru_hole circle (at 18.9 3.25) (size 1.524 1.524) (drill 0.762) (layers *.Cu *.Mask))
  (pad 9 thru_hole circle (at 18.9 8.25) (size 1.524 1.524) (drill 0.762) (layers *.Cu *.Mask))
  (pad 8 thru_hole circle (at 18.9 13.25) (size 1.524 1.524) (drill 0.762) (layers *.Cu *.Mask))
  (pad 7 thru_hole circle (at 18.9 18.25) (size 1.524 1.524) (drill 0.762) (layers *.Cu *.Mask))
  (pad 6 thru_hole circle (at 18.9 23.25) (size 1.524 1.524) (drill 0.762) (layers *.Cu *.Mask)))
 (gr_circle (center 92.5 52.5) (end 94 52.5) (layer Edge.Cuts) (width 0.1))
 (gr_circle (center 72.5 52.5) (end 74 52.5) (layer Edge.Cuts) (width 0.1))
 (gr_circle (center 72.5 32.5) (end 74 32.5) (layer Edge.Cuts) (width 0.1))
 (gr_circle (center 92.5 32.5) (end 94 32.5) (layer Edge.Cuts) (width 0.1))
 (gr_line (start 120 30) (end 55 30) (angle 90) (layer Edge.Cuts) (width 0.1))
 (gr_line (start 120 55) (end 120 30) (angle 90) (layer Edge.Cuts) (width 0.1))
 (gr_line (start 55 55) (end 120 55) (angle 90) (layer Edge.Cuts) (width 0.1))
 (gr_line (start 55 30) (end 55 55) (angle 90) (layer Edge.Cuts) (width 0.1))
 (segment (start 75.4 38) (end 79.44932 38) (width 0.25) (layer F.Cu) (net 1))
 (segment (start 79.44932 38) (end 79.94932 38.5) (width 0.25) (layer F.Cu) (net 1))
 (segment (start 75.4 46) (end 79.44932 46) (width 0.25) (layer F.Cu) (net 5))
 (segment (start 79.44932 46) (end 79.94932 46.5) (width 0.25) (layer F.Cu) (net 5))
 (segment (start 105 46.75) (end 110.5 46.75) (width 0.5) (layer B.Cu) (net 30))
 (segment (start 110.8 46.45) (end 110.8 45.05) (width 0.5) (layer B.Cu) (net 30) (status 800000))
 (segment (start 110.5 46.75) (end 110.8 46.45) (width 0.5) (layer B.Cu) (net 30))
 (via (at 104.75 46) (size 0.6) (drill 0.4) (layers F.Cu B.Cu) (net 30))
 (segment (start 104.75 46.5) (end 104.75 46) (width 0.5) (layer B.Cu) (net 30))
 (segment (start 105 46.75) (end 104.75 46.5) (width 0.5) (layer B.Cu) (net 30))
 (segment (start 101.265 47.3) (end 101.265 44.735) (width 0.5) (layer B.Cu) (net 30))
 (segment (start 101.265 44.735) (end 101.5 44.5) (width 0.5) (layer B.Cu) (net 30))
 (via (at 101.5 44.5) (size 0.6) (drill 0.4) (layers F.Cu B.Cu) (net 30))
 (segment (start 101.5 44.5) (end 103 46) (width 0.5) (layer F.Cu) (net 30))
 (segment (start 103 46) (end 104.75 46) (width 0.5) (layer F.Cu) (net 30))
 (segment (start 110.8 45.8) (end 110.8 45.05) (width 0.5) (layer B.Cu) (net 30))
 (segment (start 102.535 47.3) (end 102.535 45.435) (width 0.5) (layer B.Cu) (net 31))
 (segment (start 102.535 45.435) (end 102.5 45.4) (width 0.5) (layer B.Cu) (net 31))
 (segment (start 103.735 37.7) (end 103.735 39.735) (width 0.5) (layer B.Cu) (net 33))
 (segment (start 103.95 39.95) (end 106.2 39.95) (width 0.5) (layer B.Cu) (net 33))
 (segment (start 103.735 39.735) (end 103.95 39.95) (width 0.5) (layer B.Cu) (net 33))
 (segment (start 102.465 37.7) (end 102.465 39.565) (width 0.5) (layer B.Cu) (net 34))
 (segment (start 102.465 39.565) (end 102.5 39.6) (width 0.5) (layer B.Cu) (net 34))
 (segment (start 103.805 47.3) (end 103.805 44.195) (width 0.5) (layer B.Cu) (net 32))
 (segment (start 101.195 40.805) (end 101.195 37.7) (width 0.5) (layer B.Cu) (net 32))
 (segment (start 101 41) (end 101.195 40.805) (width 0.5) (layer B.Cu) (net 32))
 (via (at 101 41) (size 0.6) (drill 0.4) (layers F.Cu B.Cu) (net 32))
 (segment (start 104 44) (end 101 41) (width 0.5) (layer F.Cu) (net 32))
 (via (at 104 44) (size 0.6) (drill 0.4) (layers F.Cu B.Cu) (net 32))
 (segment (start 103.805 44.195) (end 104 44) (width 0.5) (layer B.Cu) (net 32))
 (segment (start 102.5 43.6) (end 103.1 43) (width 0.5) (layer B.Cu) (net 35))
 (segment (start 106.2 43.2) (end 106.2 45.05) (width 0.5) (layer B.Cu) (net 35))
 (segment (start 106 43) (end 106.2 43.2) (width 0.5) (layer B.Cu) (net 35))
 (segment (start 103.1 43) (end 106 43) (width 0.5) (layer B.Cu) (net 35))
 (segment (start 102.5 41.4) (end 103.1 42) (width 0.5) (layer B.Cu) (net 37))
 (segment (start 110.8 41.7) (end 110.8 39.95) (width 0.5) (layer B.Cu) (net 37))
 (segment (start 110.5 42) (end 110.8 41.7) (width 0.5) (layer B.Cu) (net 37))
 (segment (start 103.1 42) (end 110.5 42) (width 0.5) (layer B.Cu) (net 37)))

